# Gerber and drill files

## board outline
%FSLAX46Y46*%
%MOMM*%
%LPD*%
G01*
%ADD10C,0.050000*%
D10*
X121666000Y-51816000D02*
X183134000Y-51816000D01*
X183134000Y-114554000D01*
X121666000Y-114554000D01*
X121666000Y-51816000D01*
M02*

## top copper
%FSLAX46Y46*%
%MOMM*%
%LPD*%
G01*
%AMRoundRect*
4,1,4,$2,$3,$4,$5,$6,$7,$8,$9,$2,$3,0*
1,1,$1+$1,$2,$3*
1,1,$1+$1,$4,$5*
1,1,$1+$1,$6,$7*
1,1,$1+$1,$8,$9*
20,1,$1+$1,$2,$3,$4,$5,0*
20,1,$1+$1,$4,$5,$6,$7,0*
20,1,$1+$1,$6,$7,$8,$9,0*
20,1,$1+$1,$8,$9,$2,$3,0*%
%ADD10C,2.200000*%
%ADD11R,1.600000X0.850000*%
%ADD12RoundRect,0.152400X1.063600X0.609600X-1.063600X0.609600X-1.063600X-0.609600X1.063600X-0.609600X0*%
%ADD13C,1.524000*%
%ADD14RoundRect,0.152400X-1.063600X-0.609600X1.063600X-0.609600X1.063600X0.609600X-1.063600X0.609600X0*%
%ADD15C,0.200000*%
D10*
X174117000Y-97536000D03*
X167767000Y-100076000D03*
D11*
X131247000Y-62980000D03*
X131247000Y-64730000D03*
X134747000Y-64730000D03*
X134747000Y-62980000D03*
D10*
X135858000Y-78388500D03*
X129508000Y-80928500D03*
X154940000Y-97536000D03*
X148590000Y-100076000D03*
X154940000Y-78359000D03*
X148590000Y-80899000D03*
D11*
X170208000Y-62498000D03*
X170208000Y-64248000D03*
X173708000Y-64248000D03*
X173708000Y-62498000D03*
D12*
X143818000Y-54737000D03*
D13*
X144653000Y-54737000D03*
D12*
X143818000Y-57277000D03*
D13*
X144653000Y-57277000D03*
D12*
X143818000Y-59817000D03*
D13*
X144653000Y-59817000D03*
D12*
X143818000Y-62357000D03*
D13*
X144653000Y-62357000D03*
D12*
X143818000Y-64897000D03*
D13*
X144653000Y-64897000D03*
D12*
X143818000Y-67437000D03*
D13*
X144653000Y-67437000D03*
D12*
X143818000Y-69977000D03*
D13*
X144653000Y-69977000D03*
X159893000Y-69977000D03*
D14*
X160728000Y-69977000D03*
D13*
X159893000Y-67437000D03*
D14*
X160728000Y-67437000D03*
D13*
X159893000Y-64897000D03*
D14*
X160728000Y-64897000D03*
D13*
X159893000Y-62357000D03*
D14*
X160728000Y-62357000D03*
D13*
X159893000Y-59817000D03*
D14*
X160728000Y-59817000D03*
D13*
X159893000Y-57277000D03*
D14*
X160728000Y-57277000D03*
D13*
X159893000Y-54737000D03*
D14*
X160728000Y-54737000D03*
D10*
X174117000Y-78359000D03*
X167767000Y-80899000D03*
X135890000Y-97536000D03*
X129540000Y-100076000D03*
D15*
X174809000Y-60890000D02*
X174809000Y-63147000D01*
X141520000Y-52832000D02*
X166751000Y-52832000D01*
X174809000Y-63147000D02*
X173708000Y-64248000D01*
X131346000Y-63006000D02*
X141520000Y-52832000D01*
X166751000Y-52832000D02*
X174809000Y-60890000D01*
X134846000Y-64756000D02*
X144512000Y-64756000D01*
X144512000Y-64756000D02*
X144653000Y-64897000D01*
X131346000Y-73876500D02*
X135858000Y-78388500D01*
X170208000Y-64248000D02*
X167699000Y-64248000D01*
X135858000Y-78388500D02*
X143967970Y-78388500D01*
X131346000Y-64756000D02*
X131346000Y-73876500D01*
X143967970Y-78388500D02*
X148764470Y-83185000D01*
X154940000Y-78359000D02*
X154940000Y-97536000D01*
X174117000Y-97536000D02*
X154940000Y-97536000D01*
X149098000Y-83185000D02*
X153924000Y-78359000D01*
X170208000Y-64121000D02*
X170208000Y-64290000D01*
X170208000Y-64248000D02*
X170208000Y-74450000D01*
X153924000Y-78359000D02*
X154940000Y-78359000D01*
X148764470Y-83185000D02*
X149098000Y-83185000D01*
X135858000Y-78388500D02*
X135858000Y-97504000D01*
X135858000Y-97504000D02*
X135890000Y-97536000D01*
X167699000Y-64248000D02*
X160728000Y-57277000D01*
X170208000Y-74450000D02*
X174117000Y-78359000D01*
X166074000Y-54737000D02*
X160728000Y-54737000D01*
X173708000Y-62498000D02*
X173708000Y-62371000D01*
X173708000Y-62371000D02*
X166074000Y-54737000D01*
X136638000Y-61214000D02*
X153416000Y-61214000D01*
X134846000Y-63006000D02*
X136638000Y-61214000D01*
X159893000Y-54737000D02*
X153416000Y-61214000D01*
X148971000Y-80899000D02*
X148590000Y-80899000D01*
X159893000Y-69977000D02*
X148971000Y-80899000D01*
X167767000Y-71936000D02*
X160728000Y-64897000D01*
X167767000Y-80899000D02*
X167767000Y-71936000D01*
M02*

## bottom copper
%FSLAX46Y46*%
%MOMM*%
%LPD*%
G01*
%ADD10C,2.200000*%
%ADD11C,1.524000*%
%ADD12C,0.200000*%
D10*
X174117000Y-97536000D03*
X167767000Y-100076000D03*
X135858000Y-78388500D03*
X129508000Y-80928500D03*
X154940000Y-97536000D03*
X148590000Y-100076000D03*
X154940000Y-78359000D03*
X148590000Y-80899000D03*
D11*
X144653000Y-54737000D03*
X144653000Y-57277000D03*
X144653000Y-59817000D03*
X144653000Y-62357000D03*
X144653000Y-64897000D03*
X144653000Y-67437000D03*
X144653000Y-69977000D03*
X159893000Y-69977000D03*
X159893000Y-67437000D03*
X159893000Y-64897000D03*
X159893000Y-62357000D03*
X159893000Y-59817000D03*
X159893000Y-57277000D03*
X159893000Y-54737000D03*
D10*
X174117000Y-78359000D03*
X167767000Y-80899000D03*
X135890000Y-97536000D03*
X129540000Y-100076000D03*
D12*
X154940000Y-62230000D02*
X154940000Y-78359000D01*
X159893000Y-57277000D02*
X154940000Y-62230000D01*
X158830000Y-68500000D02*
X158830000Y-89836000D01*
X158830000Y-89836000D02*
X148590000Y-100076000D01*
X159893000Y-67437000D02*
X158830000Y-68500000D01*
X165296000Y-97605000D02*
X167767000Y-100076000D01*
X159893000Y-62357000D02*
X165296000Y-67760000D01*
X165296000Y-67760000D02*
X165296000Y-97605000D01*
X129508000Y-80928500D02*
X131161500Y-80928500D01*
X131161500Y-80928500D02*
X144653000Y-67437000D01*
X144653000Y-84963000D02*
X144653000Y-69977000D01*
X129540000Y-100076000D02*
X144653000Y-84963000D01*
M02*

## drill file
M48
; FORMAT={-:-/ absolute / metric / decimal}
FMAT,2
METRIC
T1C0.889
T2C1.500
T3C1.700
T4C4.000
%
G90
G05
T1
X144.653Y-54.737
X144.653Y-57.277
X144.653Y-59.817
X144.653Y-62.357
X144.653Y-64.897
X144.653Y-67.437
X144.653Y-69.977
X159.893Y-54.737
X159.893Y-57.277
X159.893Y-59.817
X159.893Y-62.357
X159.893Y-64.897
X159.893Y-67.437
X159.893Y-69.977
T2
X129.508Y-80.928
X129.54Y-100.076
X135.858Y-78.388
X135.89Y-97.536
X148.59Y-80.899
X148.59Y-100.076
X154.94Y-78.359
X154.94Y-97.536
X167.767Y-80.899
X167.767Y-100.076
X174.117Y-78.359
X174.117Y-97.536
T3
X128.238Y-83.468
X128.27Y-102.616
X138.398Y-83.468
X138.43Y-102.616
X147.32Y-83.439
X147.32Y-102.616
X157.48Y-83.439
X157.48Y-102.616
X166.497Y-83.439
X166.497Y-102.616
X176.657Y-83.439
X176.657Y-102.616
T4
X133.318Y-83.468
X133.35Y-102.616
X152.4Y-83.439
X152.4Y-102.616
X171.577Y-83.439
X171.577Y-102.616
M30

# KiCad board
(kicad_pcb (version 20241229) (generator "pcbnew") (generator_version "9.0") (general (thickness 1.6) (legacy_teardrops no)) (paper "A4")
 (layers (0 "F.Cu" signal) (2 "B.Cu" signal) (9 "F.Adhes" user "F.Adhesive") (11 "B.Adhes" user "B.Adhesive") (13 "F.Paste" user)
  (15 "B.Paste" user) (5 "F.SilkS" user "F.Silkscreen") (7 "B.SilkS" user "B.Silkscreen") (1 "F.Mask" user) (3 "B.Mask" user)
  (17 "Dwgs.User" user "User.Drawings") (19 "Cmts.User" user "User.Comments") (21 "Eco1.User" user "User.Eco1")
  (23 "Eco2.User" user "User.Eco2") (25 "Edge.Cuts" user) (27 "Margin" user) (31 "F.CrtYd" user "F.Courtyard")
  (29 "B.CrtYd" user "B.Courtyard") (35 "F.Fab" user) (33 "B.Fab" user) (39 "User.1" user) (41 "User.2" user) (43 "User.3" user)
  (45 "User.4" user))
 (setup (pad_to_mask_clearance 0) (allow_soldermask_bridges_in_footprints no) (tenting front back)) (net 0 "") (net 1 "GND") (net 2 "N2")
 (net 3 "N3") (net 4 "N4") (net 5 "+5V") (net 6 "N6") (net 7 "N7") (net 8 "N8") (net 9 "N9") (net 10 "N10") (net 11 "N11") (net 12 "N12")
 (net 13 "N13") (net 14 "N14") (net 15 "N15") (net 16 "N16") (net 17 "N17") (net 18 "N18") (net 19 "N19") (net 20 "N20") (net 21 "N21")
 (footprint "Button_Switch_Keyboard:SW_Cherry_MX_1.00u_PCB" (layer "F.Cu") (at 174.117 97.536)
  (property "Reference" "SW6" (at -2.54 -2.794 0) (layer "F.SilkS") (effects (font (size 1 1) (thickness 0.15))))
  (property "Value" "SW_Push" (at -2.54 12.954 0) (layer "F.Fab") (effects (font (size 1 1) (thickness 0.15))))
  (pad "" np_thru_hole circle (at -7.62 5.08) (size 1.7 1.7) (drill 1.7) (layers "*.Cu" "*.Mask"))
  (pad "" np_thru_hole circle (at -2.54 5.08) (size 4 4) (drill 4) (layers "*.Cu" "*.Mask"))
  (pad "" np_thru_hole circle (at 2.54 5.08) (size 1.7 1.7) (drill 1.7) (layers "*.Cu" "*.Mask"))
  (pad "1" thru_hole circle (at 0 0) (size 2.2 2.2) (drill 1.5) (layers "*.Cu" "*.Mask") (remove_unused_layers no) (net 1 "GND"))
  (pad "2" thru_hole circle (at -6.35 2.54) (size 2.2 2.2) (drill 1.5) (layers "*.Cu" "*.Mask") (remove_unused_layers no) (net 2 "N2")))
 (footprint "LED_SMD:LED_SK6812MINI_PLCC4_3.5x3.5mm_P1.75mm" (layer "F.Cu") (at 132.997 63.855)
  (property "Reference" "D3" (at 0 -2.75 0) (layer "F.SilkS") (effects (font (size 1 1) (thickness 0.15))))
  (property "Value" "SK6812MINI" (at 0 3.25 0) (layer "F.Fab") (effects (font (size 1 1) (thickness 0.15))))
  (pad "1" smd rect (at -1.75 -0.875) (size 1.6 0.85) (layers "F.Cu" "F.Mask" "F.Paste") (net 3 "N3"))
  (pad "2" smd rect (at -1.75 0.875) (size 1.6 0.85) (layers "F.Cu" "F.Mask" "F.Paste") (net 1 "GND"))
  (pad "3" smd rect (at 1.75 0.875) (size 1.6 0.85) (layers "F.Cu" "F.Mask" "F.Paste") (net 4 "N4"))
  (pad "4" smd rect (at 1.75 -0.875) (size 1.6 0.85) (layers "F.Cu" "F.Mask" "F.Paste") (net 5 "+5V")))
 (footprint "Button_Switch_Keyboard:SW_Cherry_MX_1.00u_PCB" (layer "F.Cu") (at 135.858 78.3885)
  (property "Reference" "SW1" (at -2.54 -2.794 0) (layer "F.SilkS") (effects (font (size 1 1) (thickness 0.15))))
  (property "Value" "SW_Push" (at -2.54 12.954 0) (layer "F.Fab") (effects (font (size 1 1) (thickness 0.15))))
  (pad "" np_thru_hole circle (at -7.62 5.08) (size 1.7 1.7) (drill 1.7) (layers "*.Cu" "*.Mask"))
  (pad "" np_thru_hole circle (at -2.54 5.08) (size 4 4) (drill 4) (layers "*.Cu" "*.Mask"))
  (pad "" np_thru_hole circle (at 2.54 5.08) (size 1.7 1.7) (drill 1.7) (layers "*.Cu" "*.Mask"))
  (pad "1" thru_hole circle (at 0 0) (size 2.2 2.2) (drill 1.5) (layers "*.Cu" "*.Mask") (remove_unused_layers no) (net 1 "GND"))
  (pad "2" thru_hole circle (at -6.35 2.54) (size 2.2 2.2) (drill 1.5) (layers "*.Cu" "*.Mask") (remove_unused_layers no) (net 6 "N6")))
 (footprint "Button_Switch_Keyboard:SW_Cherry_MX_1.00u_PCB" (layer "F.Cu") (at 154.94 97.536)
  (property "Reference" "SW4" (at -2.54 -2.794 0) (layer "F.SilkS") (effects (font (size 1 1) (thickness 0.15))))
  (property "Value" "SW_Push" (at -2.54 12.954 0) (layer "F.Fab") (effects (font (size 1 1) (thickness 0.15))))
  (pad "" np_thru_hole circle (at -7.62 5.08) (size 1.7 1.7) (drill 1.7) (layers "*.Cu" "*.Mask"))
  (pad "" np_thru_hole circle (at -2.54 5.08) (size 4 4) (drill 4) (layers "*.Cu" "*.Mask"))
  (pad "" np_thru_hole circle (at 2.54 5.08) (size 1.7 1.7) (drill 1.7) (layers "*.Cu" "*.Mask"))
  (pad "1" thru_hole circle (at 0 0) (size 2.2 2.2) (drill 1.5) (layers "*.Cu" "*.Mask") (remove_unused_layers no) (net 1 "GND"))
  (pad "2" thru_hole circle (at -6.35 2.54) (size 2.2 2.2) (drill 1.5) (layers "*.Cu" "*.Mask") (remove_unused_layers no) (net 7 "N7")))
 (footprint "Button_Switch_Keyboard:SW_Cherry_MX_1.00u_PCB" (layer "F.Cu") (at 154.94 78.359)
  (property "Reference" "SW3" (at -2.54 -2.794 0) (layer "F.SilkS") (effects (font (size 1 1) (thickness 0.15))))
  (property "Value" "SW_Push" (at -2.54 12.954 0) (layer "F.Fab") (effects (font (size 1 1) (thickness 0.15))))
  (pad "" np_thru_hole circle (at -7.62 5.08) (size 1.7 1.7) (drill 1.7) (layers "*.Cu" "*.Mask"))
  (pad "" np_thru_hole circle (at -2.54 5.08) (size 4 4) (drill 4) (layers "*.Cu" "*.Mask"))
  (pad "" np_thru_hole circle (at 2.54 5.08) (size 1.7 1.7) (drill 1.7) (layers "*.Cu" "*.Mask"))
  (pad "1" thru_hole circle (at 0 0) (size 2.2 2.2) (drill 1.5) (layers "*.Cu" "*.Mask") (remove_unused_layers no) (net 1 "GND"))
  (pad "2" thru_hole circle (at -6.35 2.54) (size 2.2 2.2) (drill 1.5) (layers "*.Cu" "*.Mask") (remove_unused_layers no) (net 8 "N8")))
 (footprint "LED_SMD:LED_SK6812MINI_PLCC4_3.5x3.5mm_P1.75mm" (layer "F.Cu") (at 171.958 63.373)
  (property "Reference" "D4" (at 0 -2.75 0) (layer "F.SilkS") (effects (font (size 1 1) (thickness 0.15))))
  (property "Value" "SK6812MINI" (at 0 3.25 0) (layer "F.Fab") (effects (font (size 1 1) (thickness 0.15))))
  (pad "1" smd rect (at -1.75 -0.875) (size 1.6 0.85) (layers "F.Cu" "F.Mask" "F.Paste") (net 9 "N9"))
  (pad "2" smd rect (at -1.75 0.875) (size 1.6 0.85) (layers "F.Cu" "F.Mask" "F.Paste") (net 1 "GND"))
  (pad "3" smd rect (at 1.75 0.875) (size 1.6 0.85) (layers "F.Cu" "F.Mask" "F.Paste") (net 3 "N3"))
  (pad "4" smd rect (at 1.75 -0.875) (size 1.6 0.85) (layers "F.Cu" "F.Mask" "F.Paste") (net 5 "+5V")))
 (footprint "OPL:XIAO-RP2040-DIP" (layer "F.Cu") (at 152.273 62.357)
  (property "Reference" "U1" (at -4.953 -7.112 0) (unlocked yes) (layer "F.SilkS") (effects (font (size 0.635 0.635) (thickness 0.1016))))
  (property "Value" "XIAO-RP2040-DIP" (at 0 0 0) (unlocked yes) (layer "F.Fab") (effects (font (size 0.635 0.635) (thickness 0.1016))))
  (pad "1" smd roundrect (at -8.455 -7.62 180) (size 2.432 1.524) (layers "F.Cu" "F.Mask") (roundrect_rratio 0.1) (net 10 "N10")
   (thermal_bridge_angle 45))
  (pad "1" thru_hole circle (at -7.62 -7.62 180) (size 1.524 1.524) (drill 0.889) (layers "*.Cu" "*.Mask") (remove_unused_layers no)
   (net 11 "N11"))
  (pad "2" smd roundrect (at -8.455 -5.08 180) (size 2.432 1.524) (layers "F.Cu" "F.Mask") (roundrect_rratio 0.1) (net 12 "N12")
   (thermal_bridge_angle 45))
  (pad "2" thru_hole circle (at -7.62 -5.08 180) (size 1.524 1.524) (drill 0.889) (layers "*.Cu" "*.Mask") (remove_unused_layers no)
   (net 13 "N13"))
  (pad "3" smd roundrect (at -8.455 -2.54 180) (size 2.432 1.524) (layers "F.Cu" "F.Mask") (roundrect_rratio 0.1) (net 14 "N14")
   (thermal_bridge_angle 45))
  (pad "3" thru_hole circle (at -7.62 -2.54 180) (size 1.524 1.524) (drill 0.889) (layers "*.Cu" "*.Mask") (remove_unused_layers no)
   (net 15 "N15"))
  (pad "4" smd roundrect (at -8.455 0 180) (size 2.432 1.524) (layers "F.Cu" "F.Mask") (roundrect_rratio 0.1) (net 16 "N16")
   (thermal_bridge_angle 45))
  (pad "4" thru_hole circle (at -7.62 0 180) (size 1.524 1.524) (drill 0.889) (layers "*.Cu" "*.Mask") (remove_unused_layers no)
   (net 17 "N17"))
  (pad "5" smd roundrect (at -8.455 2.54 180) (size 2.432 1.524) (layers "F.Cu" "F.Mask") (roundrect_rratio 0.1) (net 4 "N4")
   (thermal_bridge_angle 45))
  (pad "5" thru_hole circle (at -7.62 2.54 180) (size 1.524 1.524) (drill 0.889) (layers "*.Cu" "*.Mask") (remove_unused_layers no)
   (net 4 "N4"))
  (pad "6" smd roundrect (at -8.455 5.08 180) (size 2.432 1.524) (layers "F.Cu" "F.Mask") (roundrect_rratio 0.1) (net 6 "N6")
   (thermal_bridge_angle 45))
  (pad "6" thru_hole circle (at -7.62 5.08 180) (size 1.524 1.524) (drill 0.889) (layers "*.Cu" "*.Mask") (remove_unused_layers no)
   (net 6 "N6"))
  (pad "7" smd roundrect (at -8.455 7.62 180) (size 2.432 1.524) (layers "F.Cu" "F.Mask") (roundrect_rratio 0.1) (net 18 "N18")
   (thermal_bridge_angle 45))
  (pad "7" thru_hole circle (at -7.62 7.62 180) (size 1.524 1.524) (drill 0.889) (layers "*.Cu" "*.Mask") (remove_unused_layers no)
   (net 18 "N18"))
  (pad "8" thru_hole circle (at 7.62 7.62) (size 1.524 1.524) (drill 0.889) (layers "*.Cu" "*.Mask") (remove_unused_layers no) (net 8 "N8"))
  (pad "8" smd roundrect (at 8.455 7.62) (size 2.432 1.524) (layers "F.Cu" "F.Mask") (roundrect_rratio 0.1) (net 8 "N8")
   (thermal_bridge_angle 45))
  (pad "9" thru_hole circle (at 7.62 5.08) (size 1.524 1.524) (drill 0.889) (layers "*.Cu" "*.Mask") (remove_unused_layers no) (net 7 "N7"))
  (pad "9" smd roundrect (at 8.455 5.08) (size 2.432 1.524) (layers "F.Cu" "F.Mask") (roundrect_rratio 0.1) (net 7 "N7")
   (thermal_bridge_angle 45))
  (pad "10" thru_hole circle (at 7.62 2.54) (size 1.524 1.524) (drill 0.889) (layers "*.Cu" "*.Mask") (remove_unused_layers no)
   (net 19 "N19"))
  (pad "10" smd roundrect (at 8.455 2.54) (size 2.432 1.524) (layers "F.Cu" "F.Mask") (roundrect_rratio 0.1) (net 19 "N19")
   (thermal_bridge_angle 45))
  (pad "11" thru_hole circle (at 7.62 0) (size 1.524 1.524) (drill 0.889) (layers "*.Cu" "*.Mask") (remove_unused_layers no) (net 2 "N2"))
  (pad "11" smd roundrect (at 8.455 0) (size 2.432 1.524) (layers "F.Cu" "F.Mask") (roundrect_rratio 0.1) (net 2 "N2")
   (thermal_bridge_angle 45))
  (pad "12" thru_hole circle (at 7.62 -2.54) (size 1.524 1.524) (drill 0.889) (layers "*.Cu" "*.Mask") (remove_unused_layers no)
   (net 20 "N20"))
  (pad "12" smd roundrect (at 8.455 -2.54) (size 2.432 1.524) (layers "F.Cu" "F.Mask") (roundrect_rratio 0.1) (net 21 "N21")
   (thermal_bridge_angle 45))
  (pad "13" thru_hole circle (at 7.62 -5.08) (size 1.524 1.524) (drill 0.889) (layers "*.Cu" "*.Mask") (remove_unused_layers no)
   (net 1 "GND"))
  (pad "13" smd roundrect (at 8.455 -5.08) (size 2.432 1.524) (layers "F.Cu" "F.Mask") (roundrect_rratio 0.1) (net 1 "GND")
   (thermal_bridge_angle 45))
  (pad "14" thru_hole circle (at 7.62 -7.62) (size 1.524 1.524) (drill 0.889) (layers "*.Cu" "*.Mask") (remove_unused_layers no)
   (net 5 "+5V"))
  (pad "14" smd roundrect (at 8.455 -7.62) (size 2.432 1.524) (layers "F.Cu" "F.Mask") (roundrect_rratio 0.1) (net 5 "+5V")
   (thermal_bridge_angle 45)))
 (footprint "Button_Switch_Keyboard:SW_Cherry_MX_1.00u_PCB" (layer "F.Cu") (at 174.117 78.359)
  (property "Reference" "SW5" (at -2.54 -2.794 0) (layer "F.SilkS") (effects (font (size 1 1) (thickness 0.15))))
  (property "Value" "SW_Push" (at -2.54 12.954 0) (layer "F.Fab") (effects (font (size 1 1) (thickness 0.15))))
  (pad "" np_thru_hole circle (at -7.62 5.08) (size 1.7 1.7) (drill 1.7) (layers "*.Cu" "*.Mask"))
  (pad "" np_thru_hole circle (at -2.54 5.08) (size 4 4) (drill 4) (layers "*.Cu" "*.Mask"))
  (pad "" np_thru_hole circle (at 2.54 5.08) (size 1.7 1.7) (drill 1.7) (layers "*.Cu" "*.Mask"))
  (pad "1" thru_hole circle (at 0 0) (size 2.2 2.2) (drill 1.5) (layers "*.Cu" "*.Mask") (remove_unused_layers no) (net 1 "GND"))
  (pad "2" thru_hole circle (at -6.35 2.54) (size 2.2 2.2) (drill 1.5) (layers "*.Cu" "*.Mask") (remove_unused_layers no) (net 19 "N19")))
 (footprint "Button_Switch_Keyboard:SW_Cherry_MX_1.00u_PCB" (layer "F.Cu") (at 135.89 97.536)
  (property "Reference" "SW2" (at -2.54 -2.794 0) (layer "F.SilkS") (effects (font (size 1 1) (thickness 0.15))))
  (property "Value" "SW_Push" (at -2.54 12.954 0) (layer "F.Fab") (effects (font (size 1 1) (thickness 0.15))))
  (pad "" np_thru_hole circle (at -7.62 5.08) (size 1.7 1.7) (drill 1.7) (layers "*.Cu" "*.Mask"))
  (pad "" np_thru_hole circle (at -2.54 5.08) (size 4 4) (drill 4) (layers "*.Cu" "*.Mask"))
  (pad "" np_thru_hole circle (at 2.54 5.08) (size 1.7 1.7) (drill 1.7) (layers "*.Cu" "*.Mask"))
  (pad "1" thru_hole circle (at 0 0) (size 2.2 2.2) (drill 1.5) (layers "*.Cu" "*.Mask") (remove_unused_layers no) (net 1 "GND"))
  (pad "2" thru_hole circle (at -6.35 2.54) (size 2.2 2.2) (drill 1.5) (layers "*.Cu" "*.Mask") (remove_unused_layers no) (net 18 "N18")))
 (gr_rect (start 121.666 51.816) (end 183.134 114.554) (stroke (width 0.05) (type default)) (fill no) (layer "Edge.Cuts"))
 (segment (start 174.809 60.89) (end 174.809 63.147) (width 0.2) (layer "F.Cu") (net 3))
 (segment (start 141.52 52.832) (end 166.751 52.832) (width 0.2) (layer "F.Cu") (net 3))
 (segment (start 174.809 63.147) (end 173.708 64.248) (width 0.2) (layer "F.Cu") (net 3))
 (segment (start 131.346 63.006) (end 141.52 52.832) (width 0.2) (layer "F.Cu") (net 3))
 (segment (start 166.751 52.832) (end 174.809 60.89) (width 0.2) (layer "F.Cu") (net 3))
 (segment (start 134.846 64.756) (end 144.512 64.756) (width 0.2) (layer "F.Cu") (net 4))
 (segment (start 144.512 64.756) (end 144.653 64.897) (width 0.2) (layer "F.Cu") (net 4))
 (segment (start 131.346 73.8765) (end 135.858 78.3885) (width 0.2) (layer "F.Cu") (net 1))
 (segment (start 170.208 64.248) (end 167.699 64.248) (width 0.2) (layer "F.Cu") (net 1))
 (segment (start 135.858 78.3885) (end 143.96797 78.3885) (width 0.2) (layer "F.Cu") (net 1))
 (segment (start 131.346 64.756) (end 131.346 73.8765) (width 0.2) (layer "F.Cu") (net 1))
 (segment (start 143.96797 78.3885) (end 148.76447 83.185) (width 0.2) (layer "F.Cu") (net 1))
 (segment (start 154.94 78.359) (end 154.94 97.536) (width 0.2) (layer "F.Cu") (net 1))
 (segment (start 174.117 97.536) (end 154.94 97.536) (width 0.2) (layer "F.Cu") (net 1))
 (segment (start 149.098 83.185) (end 153.924 78.359) (width 0.2) (layer "F.Cu") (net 1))
 (segment (start 170.208 64.121) (end 170.208 64.29) (width 0.2) (layer "F.Cu") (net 1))
 (segment (start 170.208 64.248) (end 170.208 74.45) (width 0.2) (layer "F.Cu") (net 1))
 (segment (start 153.924 78.359) (end 154.94 78.359) (width 0.2) (layer "F.Cu") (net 1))
 (segment (start 148.76447 83.185) (end 149.098 83.185) (width 0.2) (layer "F.Cu") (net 1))
 (segment (start 135.858 78.3885) (end 135.858 97.504) (width 0.2) (layer "F.Cu") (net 1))
 (segment (start 135.858 97.504) (end 135.89 97.536) (width 0.2) (layer "F.Cu") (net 1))
 (segment (start 167.699 64.248) (end 160.728 57.277) (width 0.2) (layer "F.Cu") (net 1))
 (segment (start 170.208 74.45) (end 174.117 78.359) (width 0.2) (layer "F.Cu") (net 1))
 (segment (start 154.94 62.23) (end 154.94 78.359) (width 0.2) (layer "B.Cu") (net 1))
 (segment (start 159.893 57.277) (end 154.94 62.23) (width 0.2) (layer "B.Cu") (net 1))
 (segment (start 166.074 54.737) (end 160.728 54.737) (width 0.2) (layer "F.Cu") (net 5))
 (segment (start 173.708 62.498) (end 173.708 62.371) (width 0.2) (layer "F.Cu") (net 5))
 (segment (start 173.708 62.371) (end 166.074 54.737) (width 0.2) (layer "F.Cu") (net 5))
 (segment (start 136.638 61.214) (end 153.416 61.214) (width 0.2) (layer "F.Cu") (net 5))
 (segment (start 134.846 63.006) (end 136.638 61.214) (width 0.2) (layer "F.Cu") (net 5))
 (segment (start 159.893 54.737) (end 153.416 61.214) (width 0.2) (layer "F.Cu") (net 5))
 (segment (start 148.971 80.899) (end 148.59 80.899) (width 0.2) (layer "F.Cu") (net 8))
 (segment (start 159.893 69.977) (end 148.971 80.899) (width 0.2) (layer "F.Cu") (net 8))
 (segment (start 158.83 68.5) (end 158.83 89.836) (width 0.2) (layer "B.Cu") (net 7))
 (segment (start 158.83 89.836) (end 148.59 100.076) (width 0.2) (layer "B.Cu") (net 7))
 (segment (start 159.893 67.437) (end 158.83 68.5) (width 0.2) (layer "B.Cu") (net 7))
 (segment (start 167.767 71.936) (end 160.728 64.897) (width 0.2) (layer "F.Cu") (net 19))
 (segment (start 167.767 80.899) (end 167.767 71.936) (width 0.2) (layer "F.Cu") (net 19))
 (segment (start 165.296 97.605) (end 167.767 100.076) (width 0.2) (layer "B.Cu") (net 2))
 (segment (start 159.893 62.357) (end 165.296 67.76) (width 0.2) (layer "B.Cu") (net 2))
 (segment (start 165.296 67.76) (end 165.296 97.605) (width 0.2) (layer "B.Cu") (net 2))
 (segment (start 129.508 80.9285) (end 131.1615 80.9285) (width 0.2) (layer "B.Cu") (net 6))
 (segment (start 131.1615 80.9285) (end 144.653 67.437) (width 0.2) (layer "B.Cu") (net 6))
 (segment (start 144.653 84.963) (end 144.653 69.977) (width 0.2) (layer "B.Cu") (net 18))
 (segment (start 129.54 100.076) (end 144.653 84.963) (width 0.2) (layer "B.Cu") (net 18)))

